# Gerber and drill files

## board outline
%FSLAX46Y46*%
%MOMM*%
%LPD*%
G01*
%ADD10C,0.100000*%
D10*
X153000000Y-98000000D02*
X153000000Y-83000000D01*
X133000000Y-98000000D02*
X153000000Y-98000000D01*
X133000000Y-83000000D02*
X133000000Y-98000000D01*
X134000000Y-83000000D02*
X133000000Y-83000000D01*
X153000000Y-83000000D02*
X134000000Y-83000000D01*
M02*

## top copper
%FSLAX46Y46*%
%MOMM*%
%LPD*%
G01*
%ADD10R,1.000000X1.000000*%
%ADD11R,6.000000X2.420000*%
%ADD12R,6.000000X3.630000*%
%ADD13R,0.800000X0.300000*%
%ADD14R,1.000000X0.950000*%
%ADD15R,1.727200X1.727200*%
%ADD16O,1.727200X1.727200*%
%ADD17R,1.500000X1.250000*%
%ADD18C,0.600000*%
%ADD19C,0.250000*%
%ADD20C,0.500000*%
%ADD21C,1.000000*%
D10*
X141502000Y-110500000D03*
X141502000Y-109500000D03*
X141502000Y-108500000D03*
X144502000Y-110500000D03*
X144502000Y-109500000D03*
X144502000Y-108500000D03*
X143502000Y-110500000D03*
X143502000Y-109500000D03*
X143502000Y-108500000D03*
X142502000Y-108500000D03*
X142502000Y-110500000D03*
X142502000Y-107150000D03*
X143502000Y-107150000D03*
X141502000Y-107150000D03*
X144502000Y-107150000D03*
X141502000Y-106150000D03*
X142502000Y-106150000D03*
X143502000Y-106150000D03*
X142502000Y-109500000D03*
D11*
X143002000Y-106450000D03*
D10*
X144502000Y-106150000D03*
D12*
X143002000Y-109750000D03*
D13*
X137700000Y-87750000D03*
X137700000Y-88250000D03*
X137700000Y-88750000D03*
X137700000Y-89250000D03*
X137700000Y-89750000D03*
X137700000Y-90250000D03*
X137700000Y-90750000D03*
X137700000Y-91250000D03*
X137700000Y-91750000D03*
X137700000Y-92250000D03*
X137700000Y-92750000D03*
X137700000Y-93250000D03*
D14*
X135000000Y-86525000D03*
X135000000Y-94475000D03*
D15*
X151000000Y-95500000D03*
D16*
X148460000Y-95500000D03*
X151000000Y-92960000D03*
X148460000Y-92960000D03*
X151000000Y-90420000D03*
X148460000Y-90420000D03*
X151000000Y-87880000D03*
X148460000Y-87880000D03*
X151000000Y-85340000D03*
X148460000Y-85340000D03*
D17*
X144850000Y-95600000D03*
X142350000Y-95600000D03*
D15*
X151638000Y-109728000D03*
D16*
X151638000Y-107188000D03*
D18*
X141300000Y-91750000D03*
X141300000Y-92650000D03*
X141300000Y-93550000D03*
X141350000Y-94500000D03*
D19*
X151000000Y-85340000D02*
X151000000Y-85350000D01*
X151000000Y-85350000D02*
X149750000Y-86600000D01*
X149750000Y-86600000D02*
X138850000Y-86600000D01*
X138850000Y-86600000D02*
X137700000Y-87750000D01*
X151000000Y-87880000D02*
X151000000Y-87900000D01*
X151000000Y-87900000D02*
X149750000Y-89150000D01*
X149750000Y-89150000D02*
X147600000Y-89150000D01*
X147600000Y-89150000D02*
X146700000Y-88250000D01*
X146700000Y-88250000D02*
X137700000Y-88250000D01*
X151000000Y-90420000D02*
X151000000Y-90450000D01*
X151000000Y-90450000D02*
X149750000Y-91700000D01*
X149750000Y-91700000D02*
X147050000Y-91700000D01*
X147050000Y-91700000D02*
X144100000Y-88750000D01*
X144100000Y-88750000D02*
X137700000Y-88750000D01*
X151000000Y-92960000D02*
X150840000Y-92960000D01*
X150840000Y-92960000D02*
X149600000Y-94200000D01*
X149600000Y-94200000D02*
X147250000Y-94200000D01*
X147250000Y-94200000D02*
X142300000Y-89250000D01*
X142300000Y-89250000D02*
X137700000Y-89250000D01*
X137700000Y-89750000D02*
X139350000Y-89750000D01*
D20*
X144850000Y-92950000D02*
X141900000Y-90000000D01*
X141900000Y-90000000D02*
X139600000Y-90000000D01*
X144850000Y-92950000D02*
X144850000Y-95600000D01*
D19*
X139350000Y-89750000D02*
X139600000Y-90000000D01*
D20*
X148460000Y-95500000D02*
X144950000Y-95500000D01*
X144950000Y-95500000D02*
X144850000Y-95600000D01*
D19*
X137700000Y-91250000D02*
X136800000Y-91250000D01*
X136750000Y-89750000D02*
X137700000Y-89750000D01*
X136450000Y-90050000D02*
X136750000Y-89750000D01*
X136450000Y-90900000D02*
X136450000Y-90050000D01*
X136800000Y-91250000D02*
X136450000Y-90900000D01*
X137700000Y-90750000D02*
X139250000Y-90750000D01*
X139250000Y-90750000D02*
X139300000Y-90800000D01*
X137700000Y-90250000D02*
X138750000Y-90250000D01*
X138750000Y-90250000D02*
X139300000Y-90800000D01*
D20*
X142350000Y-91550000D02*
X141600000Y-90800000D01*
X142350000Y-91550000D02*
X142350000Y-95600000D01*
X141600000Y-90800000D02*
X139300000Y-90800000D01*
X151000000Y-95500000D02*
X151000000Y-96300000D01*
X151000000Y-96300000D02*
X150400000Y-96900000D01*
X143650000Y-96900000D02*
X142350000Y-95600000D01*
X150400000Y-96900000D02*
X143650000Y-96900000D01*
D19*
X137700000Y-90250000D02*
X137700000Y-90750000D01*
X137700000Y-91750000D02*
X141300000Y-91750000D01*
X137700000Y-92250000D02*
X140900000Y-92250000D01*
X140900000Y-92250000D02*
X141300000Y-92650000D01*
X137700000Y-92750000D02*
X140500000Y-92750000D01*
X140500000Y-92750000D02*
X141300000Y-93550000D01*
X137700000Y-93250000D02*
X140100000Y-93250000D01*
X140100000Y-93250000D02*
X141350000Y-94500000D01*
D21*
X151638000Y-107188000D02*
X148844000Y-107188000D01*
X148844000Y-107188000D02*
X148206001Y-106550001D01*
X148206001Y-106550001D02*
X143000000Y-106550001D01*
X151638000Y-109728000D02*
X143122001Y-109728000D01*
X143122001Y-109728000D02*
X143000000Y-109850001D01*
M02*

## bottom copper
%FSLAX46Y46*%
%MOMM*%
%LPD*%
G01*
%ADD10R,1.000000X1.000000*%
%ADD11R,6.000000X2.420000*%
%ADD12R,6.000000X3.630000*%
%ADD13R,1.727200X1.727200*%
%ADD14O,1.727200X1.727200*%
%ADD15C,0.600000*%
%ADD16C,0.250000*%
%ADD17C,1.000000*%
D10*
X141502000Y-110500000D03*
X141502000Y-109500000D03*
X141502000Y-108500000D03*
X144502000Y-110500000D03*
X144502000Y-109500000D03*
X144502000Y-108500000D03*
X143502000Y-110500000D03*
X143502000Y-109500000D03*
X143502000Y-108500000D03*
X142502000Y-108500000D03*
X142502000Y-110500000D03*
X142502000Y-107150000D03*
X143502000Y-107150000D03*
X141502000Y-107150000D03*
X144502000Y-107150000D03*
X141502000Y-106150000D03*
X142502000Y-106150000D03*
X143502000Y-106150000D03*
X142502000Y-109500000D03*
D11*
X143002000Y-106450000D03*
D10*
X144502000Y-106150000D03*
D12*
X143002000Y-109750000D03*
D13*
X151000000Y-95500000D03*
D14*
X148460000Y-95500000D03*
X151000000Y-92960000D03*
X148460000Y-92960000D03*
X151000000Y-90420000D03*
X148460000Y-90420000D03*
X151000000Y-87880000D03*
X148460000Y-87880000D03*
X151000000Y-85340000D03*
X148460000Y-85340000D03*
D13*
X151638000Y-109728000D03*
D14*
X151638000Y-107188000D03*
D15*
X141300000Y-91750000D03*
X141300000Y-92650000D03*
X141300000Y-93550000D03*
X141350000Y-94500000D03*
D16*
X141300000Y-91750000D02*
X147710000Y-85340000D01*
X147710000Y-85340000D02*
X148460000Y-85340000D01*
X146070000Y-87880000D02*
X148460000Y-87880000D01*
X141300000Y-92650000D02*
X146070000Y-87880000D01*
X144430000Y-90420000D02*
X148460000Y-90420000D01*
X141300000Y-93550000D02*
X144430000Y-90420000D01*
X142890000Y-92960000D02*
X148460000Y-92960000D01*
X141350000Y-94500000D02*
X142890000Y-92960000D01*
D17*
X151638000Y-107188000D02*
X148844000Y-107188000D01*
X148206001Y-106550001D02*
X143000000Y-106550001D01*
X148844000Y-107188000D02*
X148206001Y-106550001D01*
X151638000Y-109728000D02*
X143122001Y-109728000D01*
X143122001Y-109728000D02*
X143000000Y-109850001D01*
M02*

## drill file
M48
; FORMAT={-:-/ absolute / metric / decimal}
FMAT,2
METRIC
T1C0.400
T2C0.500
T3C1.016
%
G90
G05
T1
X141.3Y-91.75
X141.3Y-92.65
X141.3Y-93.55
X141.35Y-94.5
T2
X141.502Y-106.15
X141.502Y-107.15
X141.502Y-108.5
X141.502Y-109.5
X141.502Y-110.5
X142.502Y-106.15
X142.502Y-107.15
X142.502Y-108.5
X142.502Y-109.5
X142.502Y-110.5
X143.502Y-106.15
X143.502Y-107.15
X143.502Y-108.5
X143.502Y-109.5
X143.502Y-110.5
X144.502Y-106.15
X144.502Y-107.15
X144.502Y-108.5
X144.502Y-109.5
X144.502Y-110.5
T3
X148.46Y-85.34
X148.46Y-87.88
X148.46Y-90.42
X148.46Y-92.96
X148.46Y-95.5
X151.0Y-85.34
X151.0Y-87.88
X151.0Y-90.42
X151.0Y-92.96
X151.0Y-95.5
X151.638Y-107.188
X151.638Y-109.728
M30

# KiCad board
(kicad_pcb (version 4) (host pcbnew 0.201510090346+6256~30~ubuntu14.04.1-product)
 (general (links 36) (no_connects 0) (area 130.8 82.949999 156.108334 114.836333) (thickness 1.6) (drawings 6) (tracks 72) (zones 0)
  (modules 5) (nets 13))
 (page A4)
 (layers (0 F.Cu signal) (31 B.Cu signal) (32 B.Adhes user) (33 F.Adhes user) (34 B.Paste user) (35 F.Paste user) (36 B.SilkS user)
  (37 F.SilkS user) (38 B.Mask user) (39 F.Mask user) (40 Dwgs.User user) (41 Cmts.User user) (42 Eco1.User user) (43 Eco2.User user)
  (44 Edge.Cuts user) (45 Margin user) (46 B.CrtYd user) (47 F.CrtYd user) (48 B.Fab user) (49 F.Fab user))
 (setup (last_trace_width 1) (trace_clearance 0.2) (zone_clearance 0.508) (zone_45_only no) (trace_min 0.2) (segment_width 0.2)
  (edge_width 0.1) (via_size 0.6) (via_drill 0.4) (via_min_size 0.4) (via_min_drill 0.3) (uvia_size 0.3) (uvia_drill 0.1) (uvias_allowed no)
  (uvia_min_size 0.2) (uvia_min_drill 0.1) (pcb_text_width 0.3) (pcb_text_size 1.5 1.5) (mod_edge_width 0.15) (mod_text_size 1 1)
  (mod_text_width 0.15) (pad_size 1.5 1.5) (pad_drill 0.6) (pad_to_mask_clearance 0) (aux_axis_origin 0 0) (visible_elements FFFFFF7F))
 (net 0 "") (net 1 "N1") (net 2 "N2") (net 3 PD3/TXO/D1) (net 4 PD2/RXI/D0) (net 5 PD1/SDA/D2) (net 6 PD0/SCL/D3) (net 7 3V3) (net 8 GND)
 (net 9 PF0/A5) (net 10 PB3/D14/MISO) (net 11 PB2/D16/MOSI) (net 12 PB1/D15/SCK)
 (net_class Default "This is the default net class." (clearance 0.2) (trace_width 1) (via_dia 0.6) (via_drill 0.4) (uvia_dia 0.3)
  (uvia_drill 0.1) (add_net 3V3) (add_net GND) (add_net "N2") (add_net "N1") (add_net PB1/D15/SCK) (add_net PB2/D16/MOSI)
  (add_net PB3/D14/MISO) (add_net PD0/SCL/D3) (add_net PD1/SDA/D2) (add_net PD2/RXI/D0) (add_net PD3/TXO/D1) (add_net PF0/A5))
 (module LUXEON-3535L (layer F.Cu) (at 143.002 107.95)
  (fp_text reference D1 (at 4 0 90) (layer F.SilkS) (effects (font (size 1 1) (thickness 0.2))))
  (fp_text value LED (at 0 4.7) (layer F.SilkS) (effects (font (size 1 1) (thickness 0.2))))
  (pad 2 thru_hole rect (at -1.5 2.55) (size 1 1) (drill 0.5) (layers *.Cu *.Mask F.SilkS) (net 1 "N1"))
  (pad 2 thru_hole rect (at -1.5 1.55) (size 1 1) (drill 0.5) (layers *.Cu *.Mask F.SilkS) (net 1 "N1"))
  (pad 2 thru_hole rect (at -1.5 0.55) (size 1 1) (drill 0.5) (layers *.Cu *.Mask F.SilkS) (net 1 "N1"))
  (pad 2 thru_hole rect (at 1.5 2.55) (size 1 1) (drill 0.5) (layers *.Cu *.Mask F.SilkS) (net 1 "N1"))
  (pad 2 thru_hole rect (at 1.5 1.55) (size 1 1) (drill 0.5) (layers *.Cu *.Mask F.SilkS) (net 1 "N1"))
  (pad 2 thru_hole rect (at 1.5 0.55) (size 1 1) (drill 0.5) (layers *.Cu *.Mask F.SilkS) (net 1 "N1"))
  (pad 2 thru_hole rect (at 0.5 2.55) (size 1 1) (drill 0.5) (layers *.Cu *.Mask F.SilkS) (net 1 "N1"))
  (pad 2 thru_hole rect (at 0.5 1.55) (size 1 1) (drill 0.5) (layers *.Cu *.Mask F.SilkS) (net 1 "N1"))
  (pad 2 thru_hole rect (at 0.5 0.55) (size 1 1) (drill 0.5) (layers *.Cu *.Mask F.SilkS) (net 1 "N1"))
  (pad 2 thru_hole rect (at -0.5 0.55) (size 1 1) (drill 0.5) (layers *.Cu *.Mask F.SilkS) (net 1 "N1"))
  (pad 2 thru_hole rect (at -0.5 2.55) (size 1 1) (drill 0.5) (layers *.Cu *.Mask F.SilkS) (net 1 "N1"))
  (pad 1 thru_hole rect (at -0.5 -0.8) (size 1 1) (drill 0.5) (layers *.Cu *.Mask F.SilkS) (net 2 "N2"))
  (pad 1 thru_hole rect (at 0.5 -0.8) (size 1 1) (drill 0.5) (layers *.Cu *.Mask F.SilkS) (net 2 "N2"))
  (pad 1 thru_hole rect (at -1.5 -0.8) (size 1 1) (drill 0.5) (layers *.Cu *.Mask F.SilkS) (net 2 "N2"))
  (pad 1 thru_hole rect (at 1.5 -0.8) (size 1 1) (drill 0.5) (layers *.Cu *.Mask F.SilkS) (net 2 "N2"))
  (pad 1 thru_hole rect (at -1.5 -1.8) (size 1 1) (drill 0.5) (layers *.Cu *.Mask F.SilkS) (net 2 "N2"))
  (pad 1 thru_hole rect (at -0.5 -1.8) (size 1 1) (drill 0.5) (layers *.Cu *.Mask F.SilkS) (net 2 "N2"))
  (pad 1 thru_hole rect (at 0.5 -1.8) (size 1 1) (drill 0.5) (layers *.Cu *.Mask F.SilkS) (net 2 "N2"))
  (pad 2 thru_hole rect (at -0.5 1.55) (size 1 1) (drill 0.5) (layers *.Cu *.Mask F.SilkS) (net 1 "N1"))
  (pad 1 smd rect (at 0 -1.5) (size 6 2.42) (layers *.Cu F.SilkS) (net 2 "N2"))
  (pad 1 thru_hole rect (at 1.5 -1.8) (size 1 1) (drill 0.5) (layers *.Cu *.Mask F.SilkS) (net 2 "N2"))
  (pad 2 smd rect (at 0 1.8) (size 6 3.63) (layers *.Cu F.SilkS) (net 1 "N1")))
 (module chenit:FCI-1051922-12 (layer F.Cu) (at 135.5 90.5 270)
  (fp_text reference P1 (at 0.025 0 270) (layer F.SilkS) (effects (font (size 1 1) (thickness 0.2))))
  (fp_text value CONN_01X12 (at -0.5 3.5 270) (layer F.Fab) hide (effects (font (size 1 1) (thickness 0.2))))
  (pad 1 smd rect (at -2.75 -2.2 270) (size 0.3 0.8) (layers F.Cu F.Paste F.Mask) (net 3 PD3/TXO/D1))
  (pad 2 smd rect (at -2.25 -2.2 270) (size 0.3 0.8) (layers F.Cu F.Paste F.Mask) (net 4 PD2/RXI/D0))
  (pad 3 smd rect (at -1.75 -2.2 270) (size 0.3 0.8) (layers F.Cu F.Paste F.Mask) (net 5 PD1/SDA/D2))
  (pad 4 smd rect (at -1.25 -2.2 270) (size 0.3 0.8) (layers F.Cu F.Paste F.Mask) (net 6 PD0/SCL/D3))
  (pad 5 smd rect (at -0.75 -2.2 270) (size 0.3 0.8) (layers F.Cu F.Paste F.Mask) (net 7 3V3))
  (pad 6 smd rect (at -0.25 -2.2 270) (size 0.3 0.8) (layers F.Cu F.Paste F.Mask) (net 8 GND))
  (pad 7 smd rect (at 0.25 -2.2 270) (size 0.3 0.8) (layers F.Cu F.Paste F.Mask) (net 8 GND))
  (pad 8 smd rect (at 0.75 -2.2 270) (size 0.3 0.8) (layers F.Cu F.Paste F.Mask) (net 7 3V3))
  (pad 9 smd rect (at 1.25 -2.2 270) (size 0.3 0.8) (layers F.Cu F.Paste F.Mask) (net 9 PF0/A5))
  (pad 10 smd rect (at 1.75 -2.2 270) (size 0.3 0.8) (layers F.Cu F.Paste F.Mask) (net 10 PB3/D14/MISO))
  (pad 11 smd rect (at 2.25 -2.2 270) (size 0.3 0.8) (layers F.Cu F.Paste F.Mask) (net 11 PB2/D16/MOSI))
  (pad 12 smd rect (at 2.75 -2.2 270) (size 0.3 0.8) (layers F.Cu F.Paste F.Mask) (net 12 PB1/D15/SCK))
  (pad 13 smd rect (at -3.975 0.5 270) (size 0.95 1) (layers F.Cu F.Paste F.Mask))
  (pad 13 smd rect (at 3.975 0.5 270) (size 0.95 1) (layers F.Cu F.Paste F.Mask)))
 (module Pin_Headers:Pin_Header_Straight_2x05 (layer F.Cu) (at 151 95.5 180)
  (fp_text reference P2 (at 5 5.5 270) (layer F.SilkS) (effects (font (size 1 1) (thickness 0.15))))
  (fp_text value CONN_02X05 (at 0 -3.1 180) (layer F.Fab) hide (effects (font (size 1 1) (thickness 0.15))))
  (pad 1 thru_hole rect (at 0 0 180) (size 1.7272 1.7272) (drill 1.016) (layers *.Cu *.Mask F.SilkS) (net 8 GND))
  (pad 2 thru_hole oval (at 2.54 0 180) (size 1.7272 1.7272) (drill 1.016) (layers *.Cu *.Mask F.SilkS) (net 7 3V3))
  (pad 3 thru_hole oval (at 0 2.54 180) (size 1.7272 1.7272) (drill 1.016) (layers *.Cu *.Mask F.SilkS) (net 6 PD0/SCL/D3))
  (pad 4 thru_hole oval (at 2.54 2.54 180) (size 1.7272 1.7272) (drill 1.016) (layers *.Cu *.Mask F.SilkS) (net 12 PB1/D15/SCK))
  (pad 5 thru_hole oval (at 0 5.08 180) (size 1.7272 1.7272) (drill 1.016) (layers *.Cu *.Mask F.SilkS) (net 5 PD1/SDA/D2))
  (pad 6 thru_hole oval (at 2.54 5.08 180) (size 1.7272 1.7272) (drill 1.016) (layers *.Cu *.Mask F.SilkS) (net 11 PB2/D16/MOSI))
  (pad 7 thru_hole oval (at 0 7.62 180) (size 1.7272 1.7272) (drill 1.016) (layers *.Cu *.Mask F.SilkS) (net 4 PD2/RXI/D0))
  (pad 8 thru_hole oval (at 2.54 7.62 180) (size 1.7272 1.7272) (drill 1.016) (layers *.Cu *.Mask F.SilkS) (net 10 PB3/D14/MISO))
  (pad 9 thru_hole oval (at 0 10.16 180) (size 1.7272 1.7272) (drill 1.016) (layers *.Cu *.Mask F.SilkS) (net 3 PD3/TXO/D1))
  (pad 10 thru_hole oval (at 2.54 10.16 180) (size 1.7272 1.7272) (drill 1.016) (layers *.Cu *.Mask F.SilkS) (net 9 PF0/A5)))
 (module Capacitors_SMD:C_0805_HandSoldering (layer F.Cu) (at 143.6 95.6 180)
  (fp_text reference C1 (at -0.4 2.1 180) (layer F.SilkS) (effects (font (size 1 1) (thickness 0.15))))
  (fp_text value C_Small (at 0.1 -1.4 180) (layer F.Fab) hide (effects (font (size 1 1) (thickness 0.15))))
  (pad 1 smd rect (at -1.25 0 180) (size 1.5 1.25) (layers F.Cu F.Paste F.Mask) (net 7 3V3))
  (pad 2 smd rect (at 1.25 0 180) (size 1.5 1.25) (layers F.Cu F.Paste F.Mask) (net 8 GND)))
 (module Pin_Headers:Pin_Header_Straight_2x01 (layer F.Cu) (at 151.638 109.728 90)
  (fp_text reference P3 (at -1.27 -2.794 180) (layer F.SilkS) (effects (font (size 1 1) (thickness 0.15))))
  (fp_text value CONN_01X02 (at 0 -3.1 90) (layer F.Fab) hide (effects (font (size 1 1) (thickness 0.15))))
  (pad 1 thru_hole rect (at 0 0 90) (size 1.7272 1.7272) (drill 1.016) (layers *.Cu *.Mask F.SilkS) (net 1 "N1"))
  (pad 2 thru_hole oval (at 2.54 0 90) (size 1.7272 1.7272) (drill 1.016) (layers *.Cu *.Mask F.SilkS) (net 2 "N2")))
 (gr_line (start 153 98) (end 153 83) (angle 90) (layer Edge.Cuts) (width 0.1))
 (gr_line (start 133 98) (end 153 98) (angle 90) (layer Edge.Cuts) (width 0.1))
 (gr_line (start 133 83) (end 133 98) (angle 90) (layer Edge.Cuts) (width 0.1))
 (gr_line (start 134 83) (end 133 83) (angle 90) (layer Edge.Cuts) (width 0.1))
 (gr_line (start 153 83) (end 134 83) (angle 90) (layer Edge.Cuts) (width 0.1))
 (segment (start 151 85.34) (end 151 85.35) (width 0.25) (layer F.Cu) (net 3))
 (segment (start 151 85.35) (end 149.75 86.6) (width 0.25) (layer F.Cu) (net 3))
 (segment (start 149.75 86.6) (end 138.85 86.6) (width 0.25) (layer F.Cu) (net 3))
 (segment (start 138.85 86.6) (end 137.7 87.75) (width 0.25) (layer F.Cu) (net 3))
 (segment (start 151 87.88) (end 151 87.9) (width 0.25) (layer F.Cu) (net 4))
 (segment (start 151 87.9) (end 149.75 89.15) (width 0.25) (layer F.Cu) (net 4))
 (segment (start 149.75 89.15) (end 147.6 89.15) (width 0.25) (layer F.Cu) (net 4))
 (segment (start 147.6 89.15) (end 146.7 88.25) (width 0.25) (layer F.Cu) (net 4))
 (segment (start 146.7 88.25) (end 137.7 88.25) (width 0.25) (layer F.Cu) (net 4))
 (segment (start 151 90.42) (end 151 90.45) (width 0.25) (layer F.Cu) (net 5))
 (segment (start 151 90.45) (end 149.75 91.7) (width 0.25) (layer F.Cu) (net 5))
 (segment (start 149.75 91.7) (end 147.05 91.7) (width 0.25) (layer F.Cu) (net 5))
 (segment (start 147.05 91.7) (end 144.1 88.75) (width 0.25) (layer F.Cu) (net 5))
 (segment (start 144.1 88.75) (end 137.7 88.75) (width 0.25) (layer F.Cu) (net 5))
 (segment (start 151 92.96) (end 150.84 92.96) (width 0.25) (layer F.Cu) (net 6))
 (segment (start 150.84 92.96) (end 149.6 94.2) (width 0.25) (layer F.Cu) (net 6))
 (segment (start 149.6 94.2) (end 147.25 94.2) (width 0.25) (layer F.Cu) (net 6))
 (segment (start 147.25 94.2) (end 142.3 89.25) (width 0.25) (layer F.Cu) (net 6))
 (segment (start 142.3 89.25) (end 137.7 89.25) (width 0.25) (layer F.Cu) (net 6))
 (segment (start 137.7 89.75) (end 139.35 89.75) (width 0.25) (layer F.Cu) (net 7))
 (segment (start 144.85 92.95) (end 141.9 90) (width 0.5) (layer F.Cu) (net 7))
 (segment (start 141.9 90) (end 139.6 90) (width 0.5) (layer F.Cu) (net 7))
 (segment (start 144.85 92.95) (end 144.85 95.6) (width 0.5) (layer F.Cu) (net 7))
 (segment (start 139.35 89.75) (end 139.6 90) (width 0.25) (layer F.Cu) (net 7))
 (segment (start 148.46 95.5) (end 144.95 95.5) (width 0.5) (layer F.Cu) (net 7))
 (segment (start 144.95 95.5) (end 144.85 95.6) (width 0.5) (layer F.Cu) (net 7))
 (segment (start 137.7 91.25) (end 136.8 91.25) (width 0.25) (layer F.Cu) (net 7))
 (segment (start 136.75 89.75) (end 137.7 89.75) (width 0.25) (layer F.Cu) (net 7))
 (segment (start 136.45 90.05) (end 136.75 89.75) (width 0.25) (layer F.Cu) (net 7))
 (segment (start 136.45 90.9) (end 136.45 90.05) (width 0.25) (layer F.Cu) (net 7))
 (segment (start 136.8 91.25) (end 136.45 90.9) (width 0.25) (layer F.Cu) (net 7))
 (segment (start 137.7 90.75) (end 139.25 90.75) (width 0.25) (layer F.Cu) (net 8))
 (segment (start 139.25 90.75) (end 139.3 90.8) (width 0.25) (layer F.Cu) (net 8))
 (segment (start 137.7 90.25) (end 138.75 90.25) (width 0.25) (layer F.Cu) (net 8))
 (segment (start 138.75 90.25) (end 139.3 90.8) (width 0.25) (layer F.Cu) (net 8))
 (segment (start 142.35 91.55) (end 141.6 90.8) (width 0.5) (layer F.Cu) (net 8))
 (segment (start 142.35 91.55) (end 142.35 95.6) (width 0.5) (layer F.Cu) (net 8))
 (segment (start 141.6 90.8) (end 139.3 90.8) (width 0.5) (layer F.Cu) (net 8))
 (segment (start 151 95.5) (end 151 96.3) (width 0.5) (layer F.Cu) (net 8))
 (segment (start 151 96.3) (end 150.4 96.9) (width 0.5) (layer F.Cu) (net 8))
 (segment (start 143.65 96.9) (end 142.35 95.6) (width 0.5) (layer F.Cu) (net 8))
 (segment (start 150.4 96.9) (end 143.65 96.9) (width 0.5) (layer F.Cu) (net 8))
 (segment (start 137.7 90.25) (end 137.7 90.75) (width 0.25) (layer F.Cu) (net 8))
 (segment (start 137.7 91.75) (end 141.3 91.75) (width 0.25) (layer F.Cu) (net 9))
 (segment (start 141.3 91.75) (end 147.71 85.34) (width 0.25) (layer B.Cu) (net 9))
 (via (at 141.3 91.75) (size 0.6) (drill 0.4) (layers F.Cu B.Cu) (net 9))
 (segment (start 147.71 85.34) (end 148.46 85.34) (width 0.25) (layer B.Cu) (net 9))
 (segment (start 137.7 92.25) (end 140.9 92.25) (width 0.25) (layer F.Cu) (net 10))
 (segment (start 146.07 87.88) (end 148.46 87.88) (width 0.25) (layer B.Cu) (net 10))
 (segment (start 141.3 92.65) (end 146.07 87.88) (width 0.25) (layer B.Cu) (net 10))
 (via (at 141.3 92.65) (size 0.6) (drill 0.4) (layers F.Cu B.Cu) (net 10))
 (segment (start 140.9 92.25) (end 141.3 92.65) (width 0.25) (layer F.Cu) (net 10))
 (segment (start 137.7 92.75) (end 140.5 92.75) (width 0.25) (layer F.Cu) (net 11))
 (segment (start 144.43 90.42) (end 148.46 90.42) (width 0.25) (layer B.Cu) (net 11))
 (segment (start 141.3 93.55) (end 144.43 90.42) (width 0.25) (layer B.Cu) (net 11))
 (via (at 141.3 93.55) (size 0.6) (drill 0.4) (layers F.Cu B.Cu) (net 11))
 (segment (start 140.5 92.75) (end 141.3 93.55) (width 0.25) (layer F.Cu) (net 11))
 (segment (start 137.7 93.25) (end 140.1 93.25) (width 0.25) (layer F.Cu) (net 12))
 (segment (start 142.89 92.96) (end 148.46 92.96) (width 0.25) (layer B.Cu) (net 12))
 (segment (start 141.35 94.5) (end 142.89 92.96) (width 0.25) (layer B.Cu) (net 12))
 (via (at 141.35 94.5) (size 0.6) (drill 0.4) (layers F.Cu B.Cu) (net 12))
 (segment (start 140.1 93.25) (end 141.35 94.5) (width 0.25) (layer F.Cu) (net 12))
 (segment (start 151.638 107.188) (end 148.844 107.188) (width 1) (layer F.Cu) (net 2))
 (segment (start 148.844 107.188) (end 148.206001 106.550001) (width 1) (layer F.Cu) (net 2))
 (segment (start 148.206001 106.550001) (end 143 106.550001) (width 1) (layer F.Cu) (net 2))
 (segment (start 151.638 107.188) (end 148.844 107.188) (width 1) (layer B.Cu) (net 2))
 (segment (start 148.206001 106.550001) (end 143 106.550001) (width 1) (layer B.Cu) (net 2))
 (segment (start 148.844 107.188) (end 148.206001 106.550001) (width 1) (layer B.Cu) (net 2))
 (segment (start 151.638 109.728) (end 143.122001 109.728) (width 1) (layer F.Cu) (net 1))
 (segment (start 143.122001 109.728) (end 143 109.850001) (width 1) (layer F.Cu) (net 1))
 (segment (start 151.638 109.728) (end 143.122001 109.728) (width 1) (layer B.Cu) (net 1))
 (segment (start 143.122001 109.728) (end 143 109.850001) (width 1) (layer B.Cu) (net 1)))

